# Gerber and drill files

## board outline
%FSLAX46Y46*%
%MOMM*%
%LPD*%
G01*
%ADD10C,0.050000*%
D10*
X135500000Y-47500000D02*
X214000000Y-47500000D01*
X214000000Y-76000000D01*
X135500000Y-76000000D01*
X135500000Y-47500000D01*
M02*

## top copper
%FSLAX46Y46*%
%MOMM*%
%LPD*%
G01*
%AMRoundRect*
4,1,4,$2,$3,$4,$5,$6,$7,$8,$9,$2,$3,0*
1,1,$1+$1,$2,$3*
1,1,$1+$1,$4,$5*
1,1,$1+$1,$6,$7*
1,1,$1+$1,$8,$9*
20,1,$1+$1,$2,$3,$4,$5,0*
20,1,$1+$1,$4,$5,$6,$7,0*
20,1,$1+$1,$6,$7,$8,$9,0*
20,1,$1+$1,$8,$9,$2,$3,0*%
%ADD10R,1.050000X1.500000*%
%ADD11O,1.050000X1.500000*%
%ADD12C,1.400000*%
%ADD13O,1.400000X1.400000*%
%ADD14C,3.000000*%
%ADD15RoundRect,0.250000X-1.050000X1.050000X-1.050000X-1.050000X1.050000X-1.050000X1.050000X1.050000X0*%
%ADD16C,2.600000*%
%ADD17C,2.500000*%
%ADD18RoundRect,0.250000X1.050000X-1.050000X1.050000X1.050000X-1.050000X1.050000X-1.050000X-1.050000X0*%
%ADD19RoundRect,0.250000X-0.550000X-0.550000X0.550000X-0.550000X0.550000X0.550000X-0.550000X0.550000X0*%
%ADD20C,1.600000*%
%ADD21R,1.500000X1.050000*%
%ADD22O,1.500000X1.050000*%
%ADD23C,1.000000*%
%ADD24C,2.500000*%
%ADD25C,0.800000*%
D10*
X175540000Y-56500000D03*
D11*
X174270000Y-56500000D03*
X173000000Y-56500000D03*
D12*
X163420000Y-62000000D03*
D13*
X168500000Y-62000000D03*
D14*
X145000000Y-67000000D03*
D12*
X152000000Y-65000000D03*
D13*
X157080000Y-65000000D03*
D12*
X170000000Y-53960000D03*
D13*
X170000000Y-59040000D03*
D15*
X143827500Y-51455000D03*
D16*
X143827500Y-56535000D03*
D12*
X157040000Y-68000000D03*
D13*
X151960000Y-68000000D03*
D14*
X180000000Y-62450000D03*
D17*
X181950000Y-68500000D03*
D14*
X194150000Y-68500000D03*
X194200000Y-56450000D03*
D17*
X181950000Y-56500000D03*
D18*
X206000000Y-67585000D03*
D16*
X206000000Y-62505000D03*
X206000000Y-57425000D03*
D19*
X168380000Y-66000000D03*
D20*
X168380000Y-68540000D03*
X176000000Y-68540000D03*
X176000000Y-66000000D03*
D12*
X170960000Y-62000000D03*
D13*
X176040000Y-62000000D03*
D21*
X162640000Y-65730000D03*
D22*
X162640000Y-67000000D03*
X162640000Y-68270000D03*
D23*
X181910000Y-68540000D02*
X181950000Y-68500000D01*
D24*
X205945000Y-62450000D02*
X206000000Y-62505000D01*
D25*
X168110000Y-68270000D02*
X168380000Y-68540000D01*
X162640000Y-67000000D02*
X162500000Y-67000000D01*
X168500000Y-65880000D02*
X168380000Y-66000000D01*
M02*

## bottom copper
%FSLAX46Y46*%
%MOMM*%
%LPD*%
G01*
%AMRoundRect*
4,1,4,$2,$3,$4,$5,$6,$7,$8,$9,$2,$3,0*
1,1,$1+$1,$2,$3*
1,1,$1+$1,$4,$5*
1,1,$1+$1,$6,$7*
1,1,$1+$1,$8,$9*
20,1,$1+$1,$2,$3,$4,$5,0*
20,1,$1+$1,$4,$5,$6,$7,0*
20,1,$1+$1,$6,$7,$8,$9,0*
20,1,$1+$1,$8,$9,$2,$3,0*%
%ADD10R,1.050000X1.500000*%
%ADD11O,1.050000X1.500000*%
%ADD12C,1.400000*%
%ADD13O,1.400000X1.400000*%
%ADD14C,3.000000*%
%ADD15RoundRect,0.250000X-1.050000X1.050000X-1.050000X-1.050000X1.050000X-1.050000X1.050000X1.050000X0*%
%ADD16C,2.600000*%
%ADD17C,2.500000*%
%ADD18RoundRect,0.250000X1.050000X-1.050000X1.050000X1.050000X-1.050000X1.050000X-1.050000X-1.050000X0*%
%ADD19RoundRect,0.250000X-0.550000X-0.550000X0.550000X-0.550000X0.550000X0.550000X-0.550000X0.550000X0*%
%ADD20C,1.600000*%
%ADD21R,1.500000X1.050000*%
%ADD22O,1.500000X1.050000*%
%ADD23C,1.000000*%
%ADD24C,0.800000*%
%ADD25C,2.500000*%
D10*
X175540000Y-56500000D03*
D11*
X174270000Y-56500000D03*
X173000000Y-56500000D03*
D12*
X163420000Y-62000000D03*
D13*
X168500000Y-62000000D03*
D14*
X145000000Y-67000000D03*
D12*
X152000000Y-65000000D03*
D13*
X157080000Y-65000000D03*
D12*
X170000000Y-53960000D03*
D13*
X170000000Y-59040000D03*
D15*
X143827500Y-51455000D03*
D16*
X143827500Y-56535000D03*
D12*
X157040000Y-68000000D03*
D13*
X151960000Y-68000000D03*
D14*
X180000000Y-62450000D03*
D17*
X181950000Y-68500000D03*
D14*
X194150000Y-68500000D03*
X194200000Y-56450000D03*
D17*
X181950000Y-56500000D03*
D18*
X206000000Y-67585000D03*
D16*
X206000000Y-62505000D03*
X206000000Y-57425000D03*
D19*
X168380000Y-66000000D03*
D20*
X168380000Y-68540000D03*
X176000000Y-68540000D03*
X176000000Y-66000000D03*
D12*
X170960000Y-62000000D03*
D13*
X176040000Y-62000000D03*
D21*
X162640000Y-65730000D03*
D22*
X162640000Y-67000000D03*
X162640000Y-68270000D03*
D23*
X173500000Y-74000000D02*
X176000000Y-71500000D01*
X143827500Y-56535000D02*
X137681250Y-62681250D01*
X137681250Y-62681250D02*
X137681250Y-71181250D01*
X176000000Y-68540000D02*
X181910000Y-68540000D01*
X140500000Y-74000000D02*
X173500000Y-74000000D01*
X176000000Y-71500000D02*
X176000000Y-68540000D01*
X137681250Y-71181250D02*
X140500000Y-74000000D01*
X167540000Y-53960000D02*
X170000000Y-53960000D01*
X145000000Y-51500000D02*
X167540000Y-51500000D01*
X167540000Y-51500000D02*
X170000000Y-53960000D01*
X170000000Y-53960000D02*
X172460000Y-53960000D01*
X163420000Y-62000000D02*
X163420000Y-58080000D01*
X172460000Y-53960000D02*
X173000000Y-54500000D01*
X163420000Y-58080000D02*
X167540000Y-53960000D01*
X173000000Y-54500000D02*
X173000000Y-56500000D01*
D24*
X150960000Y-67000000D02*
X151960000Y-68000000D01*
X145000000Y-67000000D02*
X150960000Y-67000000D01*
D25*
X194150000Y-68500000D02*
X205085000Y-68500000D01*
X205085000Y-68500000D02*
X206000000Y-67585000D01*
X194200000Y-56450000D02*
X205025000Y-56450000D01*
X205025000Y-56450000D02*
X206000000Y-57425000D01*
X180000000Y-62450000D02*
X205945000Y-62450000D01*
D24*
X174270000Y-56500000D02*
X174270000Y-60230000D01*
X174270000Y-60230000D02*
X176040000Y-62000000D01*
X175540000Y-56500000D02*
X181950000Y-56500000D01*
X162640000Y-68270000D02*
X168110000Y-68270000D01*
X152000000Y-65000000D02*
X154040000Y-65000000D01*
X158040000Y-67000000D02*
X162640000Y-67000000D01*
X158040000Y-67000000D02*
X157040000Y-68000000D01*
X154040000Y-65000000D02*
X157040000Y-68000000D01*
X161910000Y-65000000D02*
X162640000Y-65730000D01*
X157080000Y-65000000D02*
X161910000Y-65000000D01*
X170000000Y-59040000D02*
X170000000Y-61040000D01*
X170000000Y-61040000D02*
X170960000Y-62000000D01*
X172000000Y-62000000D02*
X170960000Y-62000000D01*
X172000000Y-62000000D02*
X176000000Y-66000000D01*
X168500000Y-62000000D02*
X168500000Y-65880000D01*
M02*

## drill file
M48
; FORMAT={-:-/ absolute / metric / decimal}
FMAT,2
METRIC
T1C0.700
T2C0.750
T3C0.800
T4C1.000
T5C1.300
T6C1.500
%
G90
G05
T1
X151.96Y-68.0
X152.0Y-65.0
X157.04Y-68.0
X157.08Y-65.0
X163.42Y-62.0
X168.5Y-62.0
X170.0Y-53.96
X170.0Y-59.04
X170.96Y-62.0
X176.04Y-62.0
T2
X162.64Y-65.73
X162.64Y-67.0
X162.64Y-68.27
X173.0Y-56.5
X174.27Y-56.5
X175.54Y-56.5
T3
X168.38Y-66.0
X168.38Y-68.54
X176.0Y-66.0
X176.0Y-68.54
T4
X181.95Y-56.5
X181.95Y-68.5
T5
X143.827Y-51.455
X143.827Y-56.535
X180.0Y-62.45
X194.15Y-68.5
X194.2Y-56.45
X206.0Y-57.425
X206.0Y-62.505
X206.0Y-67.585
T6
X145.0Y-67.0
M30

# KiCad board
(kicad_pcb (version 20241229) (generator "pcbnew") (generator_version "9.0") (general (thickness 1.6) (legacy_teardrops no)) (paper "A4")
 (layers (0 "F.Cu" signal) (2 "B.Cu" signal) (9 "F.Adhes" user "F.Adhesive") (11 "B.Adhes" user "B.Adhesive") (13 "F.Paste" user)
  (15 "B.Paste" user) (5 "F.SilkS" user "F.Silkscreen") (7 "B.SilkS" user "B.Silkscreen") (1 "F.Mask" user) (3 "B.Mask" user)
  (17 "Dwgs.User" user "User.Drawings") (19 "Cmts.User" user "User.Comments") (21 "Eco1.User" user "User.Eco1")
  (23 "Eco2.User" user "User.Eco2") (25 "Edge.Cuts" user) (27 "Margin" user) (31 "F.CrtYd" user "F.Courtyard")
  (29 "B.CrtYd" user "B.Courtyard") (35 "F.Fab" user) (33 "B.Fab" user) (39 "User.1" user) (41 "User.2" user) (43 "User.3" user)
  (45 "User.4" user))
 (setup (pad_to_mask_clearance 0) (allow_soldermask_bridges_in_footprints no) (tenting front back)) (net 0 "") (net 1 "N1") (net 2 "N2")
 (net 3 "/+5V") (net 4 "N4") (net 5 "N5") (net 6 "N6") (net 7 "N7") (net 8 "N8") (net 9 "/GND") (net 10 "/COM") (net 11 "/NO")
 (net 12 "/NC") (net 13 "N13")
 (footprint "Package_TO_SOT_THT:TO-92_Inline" (layer "F.Cu") (at 175.54 56.5 180)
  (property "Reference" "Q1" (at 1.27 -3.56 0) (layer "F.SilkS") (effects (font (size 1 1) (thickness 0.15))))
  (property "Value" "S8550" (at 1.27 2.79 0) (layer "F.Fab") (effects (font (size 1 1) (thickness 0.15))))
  (pad "1" thru_hole rect (at 0 0 180) (size 1.05 1.5) (drill 0.75) (layers "*.Cu" "*.Mask") (remove_unused_layers no) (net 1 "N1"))
  (pad "2" thru_hole oval (at 1.27 0 180) (size 1.05 1.5) (drill 0.75) (layers "*.Cu" "*.Mask") (remove_unused_layers no) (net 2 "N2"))
  (pad "3" thru_hole oval (at 2.54 0 180) (size 1.05 1.5) (drill 0.75) (layers "*.Cu" "*.Mask") (remove_unused_layers no) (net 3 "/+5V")))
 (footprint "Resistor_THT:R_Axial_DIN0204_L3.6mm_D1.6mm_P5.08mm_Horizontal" (layer "F.Cu") (at 163.42 62)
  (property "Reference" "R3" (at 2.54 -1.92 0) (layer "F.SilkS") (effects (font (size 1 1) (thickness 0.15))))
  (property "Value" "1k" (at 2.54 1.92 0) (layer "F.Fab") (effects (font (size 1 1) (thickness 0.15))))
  (pad "1" thru_hole circle (at 0 0) (size 1.4 1.4) (drill 0.7) (layers "*.Cu" "*.Mask") (remove_unused_layers no) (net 3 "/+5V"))
  (pad "2" thru_hole oval (at 5.08 0) (size 1.4 1.4) (drill 0.7) (layers "*.Cu" "*.Mask") (remove_unused_layers no) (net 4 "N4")))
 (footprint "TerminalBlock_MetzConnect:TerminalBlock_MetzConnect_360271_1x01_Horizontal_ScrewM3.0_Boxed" (layer "F.Cu") (at 145 67)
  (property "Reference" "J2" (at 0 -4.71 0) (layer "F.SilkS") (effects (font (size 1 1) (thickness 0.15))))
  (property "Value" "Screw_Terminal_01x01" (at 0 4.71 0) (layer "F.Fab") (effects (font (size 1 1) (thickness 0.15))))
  (pad "1" thru_hole circle (at 0 0) (size 3 3) (drill 1.5) (layers "*.Cu" "*.Mask") (remove_unused_layers no) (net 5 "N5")))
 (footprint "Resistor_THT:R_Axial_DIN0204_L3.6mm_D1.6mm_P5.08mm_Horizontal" (layer "F.Cu") (at 152 65)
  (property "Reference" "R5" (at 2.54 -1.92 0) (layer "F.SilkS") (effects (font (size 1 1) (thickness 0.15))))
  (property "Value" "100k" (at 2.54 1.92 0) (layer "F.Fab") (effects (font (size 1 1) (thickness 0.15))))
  (pad "1" thru_hole circle (at 0 0) (size 1.4 1.4) (drill 0.7) (layers "*.Cu" "*.Mask") (remove_unused_layers no) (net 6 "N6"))
  (pad "2" thru_hole oval (at 5.08 0) (size 1.4 1.4) (drill 0.7) (layers "*.Cu" "*.Mask") (remove_unused_layers no) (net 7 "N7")))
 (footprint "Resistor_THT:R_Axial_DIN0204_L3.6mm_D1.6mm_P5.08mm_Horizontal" (layer "F.Cu") (at 170 53.96 -90)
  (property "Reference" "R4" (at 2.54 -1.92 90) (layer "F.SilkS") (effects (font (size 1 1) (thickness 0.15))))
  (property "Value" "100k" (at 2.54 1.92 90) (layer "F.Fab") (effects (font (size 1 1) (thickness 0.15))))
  (pad "1" thru_hole circle (at 0 0 270) (size 1.4 1.4) (drill 0.7) (layers "*.Cu" "*.Mask") (remove_unused_layers no) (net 3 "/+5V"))
  (pad "2" thru_hole oval (at 5.08 0 270) (size 1.4 1.4) (drill 0.7) (layers "*.Cu" "*.Mask") (remove_unused_layers no) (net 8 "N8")))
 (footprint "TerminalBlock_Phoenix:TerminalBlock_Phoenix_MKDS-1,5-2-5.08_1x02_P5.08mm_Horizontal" (layer "F.Cu") (at 143.8275 51.455 -90)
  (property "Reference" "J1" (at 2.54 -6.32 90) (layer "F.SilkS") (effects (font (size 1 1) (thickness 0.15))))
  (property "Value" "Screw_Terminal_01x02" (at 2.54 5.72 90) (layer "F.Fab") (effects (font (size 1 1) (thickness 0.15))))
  (pad "1" thru_hole roundrect (at 0 0 270) (size 2.6 2.6) (drill 1.3) (layers "*.Cu" "*.Mask") (remove_unused_layers no)
   (roundrect_rratio 0.096154) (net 3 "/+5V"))
  (pad "2" thru_hole circle (at 5.08 0 270) (size 2.6 2.6) (drill 1.3) (layers "*.Cu" "*.Mask") (remove_unused_layers no) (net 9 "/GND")))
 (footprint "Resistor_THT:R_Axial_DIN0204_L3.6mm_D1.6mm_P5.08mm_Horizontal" (layer "F.Cu") (at 157.04 68 180)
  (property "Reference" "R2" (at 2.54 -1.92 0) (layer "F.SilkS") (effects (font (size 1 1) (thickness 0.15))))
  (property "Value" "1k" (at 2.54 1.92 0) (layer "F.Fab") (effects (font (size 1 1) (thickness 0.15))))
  (pad "1" thru_hole circle (at 0 0 180) (size 1.4 1.4) (drill 0.7) (layers "*.Cu" "*.Mask") (remove_unused_layers no) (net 6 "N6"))
  (pad "2" thru_hole oval (at 5.08 0 180) (size 1.4 1.4) (drill 0.7) (layers "*.Cu" "*.Mask") (remove_unused_layers no) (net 5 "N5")))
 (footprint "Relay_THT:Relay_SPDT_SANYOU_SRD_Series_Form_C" (layer "F.Cu") (at 180 62.45)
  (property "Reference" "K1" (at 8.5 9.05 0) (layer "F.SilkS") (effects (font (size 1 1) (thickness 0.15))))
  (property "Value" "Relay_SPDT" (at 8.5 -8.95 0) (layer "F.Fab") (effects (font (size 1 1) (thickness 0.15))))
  (pad "1" thru_hole circle (at 0 0 90) (size 3 3) (drill 1.3) (layers "*.Cu" "*.Mask") (remove_unused_layers no) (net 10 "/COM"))
  (pad "2" thru_hole circle (at 1.95 6.05 90) (size 2.5 2.5) (drill 1) (layers "*.Cu" "*.Mask") (remove_unused_layers no) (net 9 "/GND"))
  (pad "3" thru_hole circle (at 14.15 6.05 90) (size 3 3) (drill 1.3) (layers "*.Cu" "*.Mask") (remove_unused_layers no) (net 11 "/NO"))
  (pad "4" thru_hole circle (at 14.2 -6 90) (size 3 3) (drill 1.3) (layers "*.Cu" "*.Mask") (remove_unused_layers no) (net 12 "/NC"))
  (pad "5" thru_hole circle (at 1.95 -5.95 90) (size 2.5 2.5) (drill 1) (layers "*.Cu" "*.Mask") (remove_unused_layers no) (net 1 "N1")))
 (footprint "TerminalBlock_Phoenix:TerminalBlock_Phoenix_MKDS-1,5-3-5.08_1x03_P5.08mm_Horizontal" (layer "F.Cu") (at 206 67.585 90)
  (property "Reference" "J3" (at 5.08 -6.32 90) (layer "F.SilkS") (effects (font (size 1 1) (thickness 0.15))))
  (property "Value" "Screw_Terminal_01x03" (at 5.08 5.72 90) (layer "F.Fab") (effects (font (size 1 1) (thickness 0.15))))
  (pad "1" thru_hole roundrect (at 0 0 90) (size 2.6 2.6) (drill 1.3) (layers "*.Cu" "*.Mask") (remove_unused_layers no)
   (roundrect_rratio 0.096154) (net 11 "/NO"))
  (pad "2" thru_hole circle (at 5.08 0 90) (size 2.6 2.6) (drill 1.3) (layers "*.Cu" "*.Mask") (remove_unused_layers no) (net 10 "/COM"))
  (pad "3" thru_hole circle (at 10.16 0 90) (size 2.6 2.6) (drill 1.3) (layers "*.Cu" "*.Mask") (remove_unused_layers no) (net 12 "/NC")))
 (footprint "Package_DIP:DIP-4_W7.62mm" (layer "F.Cu") (at 168.38 66)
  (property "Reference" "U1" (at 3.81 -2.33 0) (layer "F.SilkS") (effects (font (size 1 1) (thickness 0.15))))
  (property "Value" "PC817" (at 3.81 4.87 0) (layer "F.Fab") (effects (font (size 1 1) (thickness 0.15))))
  (pad "1" thru_hole roundrect (at 0 0) (size 1.6 1.6) (drill 0.8) (layers "*.Cu" "*.Mask") (remove_unused_layers no)
   (roundrect_rratio 0.15625) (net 4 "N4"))
  (pad "2" thru_hole circle (at 0 2.54) (size 1.6 1.6) (drill 0.8) (layers "*.Cu" "*.Mask") (remove_unused_layers no) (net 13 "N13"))
  (pad "3" thru_hole circle (at 7.62 2.54) (size 1.6 1.6) (drill 0.8) (layers "*.Cu" "*.Mask") (remove_unused_layers no) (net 9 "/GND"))
  (pad "4" thru_hole circle (at 7.62 0) (size 1.6 1.6) (drill 0.8) (layers "*.Cu" "*.Mask") (remove_unused_layers no) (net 8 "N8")))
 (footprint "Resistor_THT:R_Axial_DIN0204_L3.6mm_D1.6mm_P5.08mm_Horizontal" (layer "F.Cu") (at 170.96 62)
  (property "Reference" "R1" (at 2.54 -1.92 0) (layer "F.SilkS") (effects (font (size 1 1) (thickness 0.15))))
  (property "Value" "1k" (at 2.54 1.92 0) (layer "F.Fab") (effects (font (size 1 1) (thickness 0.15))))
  (pad "1" thru_hole circle (at 0 0) (size 1.4 1.4) (drill 0.7) (layers "*.Cu" "*.Mask") (remove_unused_layers no) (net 8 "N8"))
  (pad "2" thru_hole oval (at 5.08 0) (size 1.4 1.4) (drill 0.7) (layers "*.Cu" "*.Mask") (remove_unused_layers no) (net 2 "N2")))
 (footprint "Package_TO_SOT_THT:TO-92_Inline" (layer "F.Cu") (at 162.64 65.73 -90)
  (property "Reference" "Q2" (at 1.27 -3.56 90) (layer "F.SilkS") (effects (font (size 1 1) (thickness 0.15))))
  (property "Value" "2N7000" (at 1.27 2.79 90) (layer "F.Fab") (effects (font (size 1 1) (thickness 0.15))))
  (pad "1" thru_hole rect (at 0 0 270) (size 1.05 1.5) (drill 0.75) (layers "*.Cu" "*.Mask") (remove_unused_layers no) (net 7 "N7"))
  (pad "2" thru_hole oval (at 1.27 0 270) (size 1.05 1.5) (drill 0.75) (layers "*.Cu" "*.Mask") (remove_unused_layers no) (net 6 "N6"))
  (pad "3" thru_hole oval (at 2.54 0 270) (size 1.05 1.5) (drill 0.75) (layers "*.Cu" "*.Mask") (remove_unused_layers no) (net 13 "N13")))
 (gr_rect (start 135.5 47.5) (end 214 76) (stroke (width 0.05) (type default)) (fill no) (layer "Edge.Cuts"))
 (segment (start 181.91 68.54) (end 181.95 68.5) (width 1) (layer "F.Cu") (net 9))
 (segment (start 173.5 74) (end 176 71.5) (width 1) (layer "B.Cu") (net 9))
 (segment (start 143.8275 56.535) (end 137.68125 62.68125) (width 1) (layer "B.Cu") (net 9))
 (segment (start 137.68125 62.68125) (end 137.68125 71.18125) (width 1) (layer "B.Cu") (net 9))
 (segment (start 176 68.54) (end 181.91 68.54) (width 1) (layer "B.Cu") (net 9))
 (segment (start 140.5 74) (end 173.5 74) (width 1) (layer "B.Cu") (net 9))
 (segment (start 176 71.5) (end 176 68.54) (width 1) (layer "B.Cu") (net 9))
 (segment (start 137.68125 71.18125) (end 140.5 74) (width 1) (layer "B.Cu") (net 9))
 (segment (start 167.54 53.96) (end 170 53.96) (width 1) (layer "B.Cu") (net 3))
 (segment (start 145 51.5) (end 167.54 51.5) (width 1) (layer "B.Cu") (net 3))
 (segment (start 167.54 51.5) (end 170 53.96) (width 1) (layer "B.Cu") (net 3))
 (segment (start 170 53.96) (end 172.46 53.96) (width 1) (layer "B.Cu") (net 3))
 (segment (start 163.42 62) (end 163.42 58.08) (width 1) (layer "B.Cu") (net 3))
 (segment (start 172.46 53.96) (end 173 54.5) (width 1) (layer "B.Cu") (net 3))
 (segment (start 163.42 58.08) (end 167.54 53.96) (width 1) (layer "B.Cu") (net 3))
 (segment (start 173 54.5) (end 173 56.5) (width 1) (layer "B.Cu") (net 3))
 (segment (start 150.96 67) (end 151.96 68) (width 0.8) (layer "B.Cu") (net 5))
 (segment (start 145 67) (end 150.96 67) (width 0.8) (layer "B.Cu") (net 5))
 (segment (start 194.15 68.5) (end 205.085 68.5) (width 2.5) (layer "B.Cu") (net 11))
 (segment (start 205.085 68.5) (end 206 67.585) (width 2.5) (layer "B.Cu") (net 11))
 (segment (start 194.2 56.45) (end 205.025 56.45) (width 2.5) (layer "B.Cu") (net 12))
 (segment (start 205.025 56.45) (end 206 57.425) (width 2.5) (layer "B.Cu") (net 12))
 (segment (start 205.945 62.45) (end 206 62.505) (width 2.5) (layer "F.Cu") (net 10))
 (segment (start 180 62.45) (end 205.945 62.45) (width 2.5) (layer "B.Cu") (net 10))
 (segment (start 174.27 56.5) (end 174.27 60.23) (width 0.8) (layer "B.Cu") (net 2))
 (segment (start 174.27 60.23) (end 176.04 62) (width 0.8) (layer "B.Cu") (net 2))
 (segment (start 175.54 56.5) (end 181.95 56.5) (width 0.8) (layer "B.Cu") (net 1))
 (segment (start 168.11 68.27) (end 168.38 68.54) (width 0.8) (layer "F.Cu") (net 13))
 (segment (start 162.64 68.27) (end 168.11 68.27) (width 0.8) (layer "B.Cu") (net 13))
 (segment (start 162.64 67) (end 162.5 67) (width 0.8) (layer "F.Cu") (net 6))
 (segment (start 152 65) (end 154.04 65) (width 0.8) (layer "B.Cu") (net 6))
 (segment (start 158.04 67) (end 162.64 67) (width 0.8) (layer "B.Cu") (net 6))
 (segment (start 158.04 67) (end 157.04 68) (width 0.8) (layer "B.Cu") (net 6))
 (segment (start 154.04 65) (end 157.04 68) (width 0.8) (layer "B.Cu") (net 6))
 (segment (start 161.91 65) (end 162.64 65.73) (width 0.8) (layer "B.Cu") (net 7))
 (segment (start 157.08 65) (end 161.91 65) (width 0.8) (layer "B.Cu") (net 7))
 (segment (start 170 59.04) (end 170 61.04) (width 0.8) (layer "B.Cu") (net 8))
 (segment (start 170 61.04) (end 170.96 62) (width 0.8) (layer "B.Cu") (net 8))
 (segment (start 172 62) (end 170.96 62) (width 0.8) (layer "B.Cu") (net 8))
 (segment (start 172 62) (end 176 66) (width 0.8) (layer "B.Cu") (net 8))
 (segment (start 168.5 65.88) (end 168.38 66) (width 0.8) (layer "F.Cu") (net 4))
 (segment (start 168.5 62) (end 168.5 65.88) (width 0.8) (layer "B.Cu") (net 4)))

